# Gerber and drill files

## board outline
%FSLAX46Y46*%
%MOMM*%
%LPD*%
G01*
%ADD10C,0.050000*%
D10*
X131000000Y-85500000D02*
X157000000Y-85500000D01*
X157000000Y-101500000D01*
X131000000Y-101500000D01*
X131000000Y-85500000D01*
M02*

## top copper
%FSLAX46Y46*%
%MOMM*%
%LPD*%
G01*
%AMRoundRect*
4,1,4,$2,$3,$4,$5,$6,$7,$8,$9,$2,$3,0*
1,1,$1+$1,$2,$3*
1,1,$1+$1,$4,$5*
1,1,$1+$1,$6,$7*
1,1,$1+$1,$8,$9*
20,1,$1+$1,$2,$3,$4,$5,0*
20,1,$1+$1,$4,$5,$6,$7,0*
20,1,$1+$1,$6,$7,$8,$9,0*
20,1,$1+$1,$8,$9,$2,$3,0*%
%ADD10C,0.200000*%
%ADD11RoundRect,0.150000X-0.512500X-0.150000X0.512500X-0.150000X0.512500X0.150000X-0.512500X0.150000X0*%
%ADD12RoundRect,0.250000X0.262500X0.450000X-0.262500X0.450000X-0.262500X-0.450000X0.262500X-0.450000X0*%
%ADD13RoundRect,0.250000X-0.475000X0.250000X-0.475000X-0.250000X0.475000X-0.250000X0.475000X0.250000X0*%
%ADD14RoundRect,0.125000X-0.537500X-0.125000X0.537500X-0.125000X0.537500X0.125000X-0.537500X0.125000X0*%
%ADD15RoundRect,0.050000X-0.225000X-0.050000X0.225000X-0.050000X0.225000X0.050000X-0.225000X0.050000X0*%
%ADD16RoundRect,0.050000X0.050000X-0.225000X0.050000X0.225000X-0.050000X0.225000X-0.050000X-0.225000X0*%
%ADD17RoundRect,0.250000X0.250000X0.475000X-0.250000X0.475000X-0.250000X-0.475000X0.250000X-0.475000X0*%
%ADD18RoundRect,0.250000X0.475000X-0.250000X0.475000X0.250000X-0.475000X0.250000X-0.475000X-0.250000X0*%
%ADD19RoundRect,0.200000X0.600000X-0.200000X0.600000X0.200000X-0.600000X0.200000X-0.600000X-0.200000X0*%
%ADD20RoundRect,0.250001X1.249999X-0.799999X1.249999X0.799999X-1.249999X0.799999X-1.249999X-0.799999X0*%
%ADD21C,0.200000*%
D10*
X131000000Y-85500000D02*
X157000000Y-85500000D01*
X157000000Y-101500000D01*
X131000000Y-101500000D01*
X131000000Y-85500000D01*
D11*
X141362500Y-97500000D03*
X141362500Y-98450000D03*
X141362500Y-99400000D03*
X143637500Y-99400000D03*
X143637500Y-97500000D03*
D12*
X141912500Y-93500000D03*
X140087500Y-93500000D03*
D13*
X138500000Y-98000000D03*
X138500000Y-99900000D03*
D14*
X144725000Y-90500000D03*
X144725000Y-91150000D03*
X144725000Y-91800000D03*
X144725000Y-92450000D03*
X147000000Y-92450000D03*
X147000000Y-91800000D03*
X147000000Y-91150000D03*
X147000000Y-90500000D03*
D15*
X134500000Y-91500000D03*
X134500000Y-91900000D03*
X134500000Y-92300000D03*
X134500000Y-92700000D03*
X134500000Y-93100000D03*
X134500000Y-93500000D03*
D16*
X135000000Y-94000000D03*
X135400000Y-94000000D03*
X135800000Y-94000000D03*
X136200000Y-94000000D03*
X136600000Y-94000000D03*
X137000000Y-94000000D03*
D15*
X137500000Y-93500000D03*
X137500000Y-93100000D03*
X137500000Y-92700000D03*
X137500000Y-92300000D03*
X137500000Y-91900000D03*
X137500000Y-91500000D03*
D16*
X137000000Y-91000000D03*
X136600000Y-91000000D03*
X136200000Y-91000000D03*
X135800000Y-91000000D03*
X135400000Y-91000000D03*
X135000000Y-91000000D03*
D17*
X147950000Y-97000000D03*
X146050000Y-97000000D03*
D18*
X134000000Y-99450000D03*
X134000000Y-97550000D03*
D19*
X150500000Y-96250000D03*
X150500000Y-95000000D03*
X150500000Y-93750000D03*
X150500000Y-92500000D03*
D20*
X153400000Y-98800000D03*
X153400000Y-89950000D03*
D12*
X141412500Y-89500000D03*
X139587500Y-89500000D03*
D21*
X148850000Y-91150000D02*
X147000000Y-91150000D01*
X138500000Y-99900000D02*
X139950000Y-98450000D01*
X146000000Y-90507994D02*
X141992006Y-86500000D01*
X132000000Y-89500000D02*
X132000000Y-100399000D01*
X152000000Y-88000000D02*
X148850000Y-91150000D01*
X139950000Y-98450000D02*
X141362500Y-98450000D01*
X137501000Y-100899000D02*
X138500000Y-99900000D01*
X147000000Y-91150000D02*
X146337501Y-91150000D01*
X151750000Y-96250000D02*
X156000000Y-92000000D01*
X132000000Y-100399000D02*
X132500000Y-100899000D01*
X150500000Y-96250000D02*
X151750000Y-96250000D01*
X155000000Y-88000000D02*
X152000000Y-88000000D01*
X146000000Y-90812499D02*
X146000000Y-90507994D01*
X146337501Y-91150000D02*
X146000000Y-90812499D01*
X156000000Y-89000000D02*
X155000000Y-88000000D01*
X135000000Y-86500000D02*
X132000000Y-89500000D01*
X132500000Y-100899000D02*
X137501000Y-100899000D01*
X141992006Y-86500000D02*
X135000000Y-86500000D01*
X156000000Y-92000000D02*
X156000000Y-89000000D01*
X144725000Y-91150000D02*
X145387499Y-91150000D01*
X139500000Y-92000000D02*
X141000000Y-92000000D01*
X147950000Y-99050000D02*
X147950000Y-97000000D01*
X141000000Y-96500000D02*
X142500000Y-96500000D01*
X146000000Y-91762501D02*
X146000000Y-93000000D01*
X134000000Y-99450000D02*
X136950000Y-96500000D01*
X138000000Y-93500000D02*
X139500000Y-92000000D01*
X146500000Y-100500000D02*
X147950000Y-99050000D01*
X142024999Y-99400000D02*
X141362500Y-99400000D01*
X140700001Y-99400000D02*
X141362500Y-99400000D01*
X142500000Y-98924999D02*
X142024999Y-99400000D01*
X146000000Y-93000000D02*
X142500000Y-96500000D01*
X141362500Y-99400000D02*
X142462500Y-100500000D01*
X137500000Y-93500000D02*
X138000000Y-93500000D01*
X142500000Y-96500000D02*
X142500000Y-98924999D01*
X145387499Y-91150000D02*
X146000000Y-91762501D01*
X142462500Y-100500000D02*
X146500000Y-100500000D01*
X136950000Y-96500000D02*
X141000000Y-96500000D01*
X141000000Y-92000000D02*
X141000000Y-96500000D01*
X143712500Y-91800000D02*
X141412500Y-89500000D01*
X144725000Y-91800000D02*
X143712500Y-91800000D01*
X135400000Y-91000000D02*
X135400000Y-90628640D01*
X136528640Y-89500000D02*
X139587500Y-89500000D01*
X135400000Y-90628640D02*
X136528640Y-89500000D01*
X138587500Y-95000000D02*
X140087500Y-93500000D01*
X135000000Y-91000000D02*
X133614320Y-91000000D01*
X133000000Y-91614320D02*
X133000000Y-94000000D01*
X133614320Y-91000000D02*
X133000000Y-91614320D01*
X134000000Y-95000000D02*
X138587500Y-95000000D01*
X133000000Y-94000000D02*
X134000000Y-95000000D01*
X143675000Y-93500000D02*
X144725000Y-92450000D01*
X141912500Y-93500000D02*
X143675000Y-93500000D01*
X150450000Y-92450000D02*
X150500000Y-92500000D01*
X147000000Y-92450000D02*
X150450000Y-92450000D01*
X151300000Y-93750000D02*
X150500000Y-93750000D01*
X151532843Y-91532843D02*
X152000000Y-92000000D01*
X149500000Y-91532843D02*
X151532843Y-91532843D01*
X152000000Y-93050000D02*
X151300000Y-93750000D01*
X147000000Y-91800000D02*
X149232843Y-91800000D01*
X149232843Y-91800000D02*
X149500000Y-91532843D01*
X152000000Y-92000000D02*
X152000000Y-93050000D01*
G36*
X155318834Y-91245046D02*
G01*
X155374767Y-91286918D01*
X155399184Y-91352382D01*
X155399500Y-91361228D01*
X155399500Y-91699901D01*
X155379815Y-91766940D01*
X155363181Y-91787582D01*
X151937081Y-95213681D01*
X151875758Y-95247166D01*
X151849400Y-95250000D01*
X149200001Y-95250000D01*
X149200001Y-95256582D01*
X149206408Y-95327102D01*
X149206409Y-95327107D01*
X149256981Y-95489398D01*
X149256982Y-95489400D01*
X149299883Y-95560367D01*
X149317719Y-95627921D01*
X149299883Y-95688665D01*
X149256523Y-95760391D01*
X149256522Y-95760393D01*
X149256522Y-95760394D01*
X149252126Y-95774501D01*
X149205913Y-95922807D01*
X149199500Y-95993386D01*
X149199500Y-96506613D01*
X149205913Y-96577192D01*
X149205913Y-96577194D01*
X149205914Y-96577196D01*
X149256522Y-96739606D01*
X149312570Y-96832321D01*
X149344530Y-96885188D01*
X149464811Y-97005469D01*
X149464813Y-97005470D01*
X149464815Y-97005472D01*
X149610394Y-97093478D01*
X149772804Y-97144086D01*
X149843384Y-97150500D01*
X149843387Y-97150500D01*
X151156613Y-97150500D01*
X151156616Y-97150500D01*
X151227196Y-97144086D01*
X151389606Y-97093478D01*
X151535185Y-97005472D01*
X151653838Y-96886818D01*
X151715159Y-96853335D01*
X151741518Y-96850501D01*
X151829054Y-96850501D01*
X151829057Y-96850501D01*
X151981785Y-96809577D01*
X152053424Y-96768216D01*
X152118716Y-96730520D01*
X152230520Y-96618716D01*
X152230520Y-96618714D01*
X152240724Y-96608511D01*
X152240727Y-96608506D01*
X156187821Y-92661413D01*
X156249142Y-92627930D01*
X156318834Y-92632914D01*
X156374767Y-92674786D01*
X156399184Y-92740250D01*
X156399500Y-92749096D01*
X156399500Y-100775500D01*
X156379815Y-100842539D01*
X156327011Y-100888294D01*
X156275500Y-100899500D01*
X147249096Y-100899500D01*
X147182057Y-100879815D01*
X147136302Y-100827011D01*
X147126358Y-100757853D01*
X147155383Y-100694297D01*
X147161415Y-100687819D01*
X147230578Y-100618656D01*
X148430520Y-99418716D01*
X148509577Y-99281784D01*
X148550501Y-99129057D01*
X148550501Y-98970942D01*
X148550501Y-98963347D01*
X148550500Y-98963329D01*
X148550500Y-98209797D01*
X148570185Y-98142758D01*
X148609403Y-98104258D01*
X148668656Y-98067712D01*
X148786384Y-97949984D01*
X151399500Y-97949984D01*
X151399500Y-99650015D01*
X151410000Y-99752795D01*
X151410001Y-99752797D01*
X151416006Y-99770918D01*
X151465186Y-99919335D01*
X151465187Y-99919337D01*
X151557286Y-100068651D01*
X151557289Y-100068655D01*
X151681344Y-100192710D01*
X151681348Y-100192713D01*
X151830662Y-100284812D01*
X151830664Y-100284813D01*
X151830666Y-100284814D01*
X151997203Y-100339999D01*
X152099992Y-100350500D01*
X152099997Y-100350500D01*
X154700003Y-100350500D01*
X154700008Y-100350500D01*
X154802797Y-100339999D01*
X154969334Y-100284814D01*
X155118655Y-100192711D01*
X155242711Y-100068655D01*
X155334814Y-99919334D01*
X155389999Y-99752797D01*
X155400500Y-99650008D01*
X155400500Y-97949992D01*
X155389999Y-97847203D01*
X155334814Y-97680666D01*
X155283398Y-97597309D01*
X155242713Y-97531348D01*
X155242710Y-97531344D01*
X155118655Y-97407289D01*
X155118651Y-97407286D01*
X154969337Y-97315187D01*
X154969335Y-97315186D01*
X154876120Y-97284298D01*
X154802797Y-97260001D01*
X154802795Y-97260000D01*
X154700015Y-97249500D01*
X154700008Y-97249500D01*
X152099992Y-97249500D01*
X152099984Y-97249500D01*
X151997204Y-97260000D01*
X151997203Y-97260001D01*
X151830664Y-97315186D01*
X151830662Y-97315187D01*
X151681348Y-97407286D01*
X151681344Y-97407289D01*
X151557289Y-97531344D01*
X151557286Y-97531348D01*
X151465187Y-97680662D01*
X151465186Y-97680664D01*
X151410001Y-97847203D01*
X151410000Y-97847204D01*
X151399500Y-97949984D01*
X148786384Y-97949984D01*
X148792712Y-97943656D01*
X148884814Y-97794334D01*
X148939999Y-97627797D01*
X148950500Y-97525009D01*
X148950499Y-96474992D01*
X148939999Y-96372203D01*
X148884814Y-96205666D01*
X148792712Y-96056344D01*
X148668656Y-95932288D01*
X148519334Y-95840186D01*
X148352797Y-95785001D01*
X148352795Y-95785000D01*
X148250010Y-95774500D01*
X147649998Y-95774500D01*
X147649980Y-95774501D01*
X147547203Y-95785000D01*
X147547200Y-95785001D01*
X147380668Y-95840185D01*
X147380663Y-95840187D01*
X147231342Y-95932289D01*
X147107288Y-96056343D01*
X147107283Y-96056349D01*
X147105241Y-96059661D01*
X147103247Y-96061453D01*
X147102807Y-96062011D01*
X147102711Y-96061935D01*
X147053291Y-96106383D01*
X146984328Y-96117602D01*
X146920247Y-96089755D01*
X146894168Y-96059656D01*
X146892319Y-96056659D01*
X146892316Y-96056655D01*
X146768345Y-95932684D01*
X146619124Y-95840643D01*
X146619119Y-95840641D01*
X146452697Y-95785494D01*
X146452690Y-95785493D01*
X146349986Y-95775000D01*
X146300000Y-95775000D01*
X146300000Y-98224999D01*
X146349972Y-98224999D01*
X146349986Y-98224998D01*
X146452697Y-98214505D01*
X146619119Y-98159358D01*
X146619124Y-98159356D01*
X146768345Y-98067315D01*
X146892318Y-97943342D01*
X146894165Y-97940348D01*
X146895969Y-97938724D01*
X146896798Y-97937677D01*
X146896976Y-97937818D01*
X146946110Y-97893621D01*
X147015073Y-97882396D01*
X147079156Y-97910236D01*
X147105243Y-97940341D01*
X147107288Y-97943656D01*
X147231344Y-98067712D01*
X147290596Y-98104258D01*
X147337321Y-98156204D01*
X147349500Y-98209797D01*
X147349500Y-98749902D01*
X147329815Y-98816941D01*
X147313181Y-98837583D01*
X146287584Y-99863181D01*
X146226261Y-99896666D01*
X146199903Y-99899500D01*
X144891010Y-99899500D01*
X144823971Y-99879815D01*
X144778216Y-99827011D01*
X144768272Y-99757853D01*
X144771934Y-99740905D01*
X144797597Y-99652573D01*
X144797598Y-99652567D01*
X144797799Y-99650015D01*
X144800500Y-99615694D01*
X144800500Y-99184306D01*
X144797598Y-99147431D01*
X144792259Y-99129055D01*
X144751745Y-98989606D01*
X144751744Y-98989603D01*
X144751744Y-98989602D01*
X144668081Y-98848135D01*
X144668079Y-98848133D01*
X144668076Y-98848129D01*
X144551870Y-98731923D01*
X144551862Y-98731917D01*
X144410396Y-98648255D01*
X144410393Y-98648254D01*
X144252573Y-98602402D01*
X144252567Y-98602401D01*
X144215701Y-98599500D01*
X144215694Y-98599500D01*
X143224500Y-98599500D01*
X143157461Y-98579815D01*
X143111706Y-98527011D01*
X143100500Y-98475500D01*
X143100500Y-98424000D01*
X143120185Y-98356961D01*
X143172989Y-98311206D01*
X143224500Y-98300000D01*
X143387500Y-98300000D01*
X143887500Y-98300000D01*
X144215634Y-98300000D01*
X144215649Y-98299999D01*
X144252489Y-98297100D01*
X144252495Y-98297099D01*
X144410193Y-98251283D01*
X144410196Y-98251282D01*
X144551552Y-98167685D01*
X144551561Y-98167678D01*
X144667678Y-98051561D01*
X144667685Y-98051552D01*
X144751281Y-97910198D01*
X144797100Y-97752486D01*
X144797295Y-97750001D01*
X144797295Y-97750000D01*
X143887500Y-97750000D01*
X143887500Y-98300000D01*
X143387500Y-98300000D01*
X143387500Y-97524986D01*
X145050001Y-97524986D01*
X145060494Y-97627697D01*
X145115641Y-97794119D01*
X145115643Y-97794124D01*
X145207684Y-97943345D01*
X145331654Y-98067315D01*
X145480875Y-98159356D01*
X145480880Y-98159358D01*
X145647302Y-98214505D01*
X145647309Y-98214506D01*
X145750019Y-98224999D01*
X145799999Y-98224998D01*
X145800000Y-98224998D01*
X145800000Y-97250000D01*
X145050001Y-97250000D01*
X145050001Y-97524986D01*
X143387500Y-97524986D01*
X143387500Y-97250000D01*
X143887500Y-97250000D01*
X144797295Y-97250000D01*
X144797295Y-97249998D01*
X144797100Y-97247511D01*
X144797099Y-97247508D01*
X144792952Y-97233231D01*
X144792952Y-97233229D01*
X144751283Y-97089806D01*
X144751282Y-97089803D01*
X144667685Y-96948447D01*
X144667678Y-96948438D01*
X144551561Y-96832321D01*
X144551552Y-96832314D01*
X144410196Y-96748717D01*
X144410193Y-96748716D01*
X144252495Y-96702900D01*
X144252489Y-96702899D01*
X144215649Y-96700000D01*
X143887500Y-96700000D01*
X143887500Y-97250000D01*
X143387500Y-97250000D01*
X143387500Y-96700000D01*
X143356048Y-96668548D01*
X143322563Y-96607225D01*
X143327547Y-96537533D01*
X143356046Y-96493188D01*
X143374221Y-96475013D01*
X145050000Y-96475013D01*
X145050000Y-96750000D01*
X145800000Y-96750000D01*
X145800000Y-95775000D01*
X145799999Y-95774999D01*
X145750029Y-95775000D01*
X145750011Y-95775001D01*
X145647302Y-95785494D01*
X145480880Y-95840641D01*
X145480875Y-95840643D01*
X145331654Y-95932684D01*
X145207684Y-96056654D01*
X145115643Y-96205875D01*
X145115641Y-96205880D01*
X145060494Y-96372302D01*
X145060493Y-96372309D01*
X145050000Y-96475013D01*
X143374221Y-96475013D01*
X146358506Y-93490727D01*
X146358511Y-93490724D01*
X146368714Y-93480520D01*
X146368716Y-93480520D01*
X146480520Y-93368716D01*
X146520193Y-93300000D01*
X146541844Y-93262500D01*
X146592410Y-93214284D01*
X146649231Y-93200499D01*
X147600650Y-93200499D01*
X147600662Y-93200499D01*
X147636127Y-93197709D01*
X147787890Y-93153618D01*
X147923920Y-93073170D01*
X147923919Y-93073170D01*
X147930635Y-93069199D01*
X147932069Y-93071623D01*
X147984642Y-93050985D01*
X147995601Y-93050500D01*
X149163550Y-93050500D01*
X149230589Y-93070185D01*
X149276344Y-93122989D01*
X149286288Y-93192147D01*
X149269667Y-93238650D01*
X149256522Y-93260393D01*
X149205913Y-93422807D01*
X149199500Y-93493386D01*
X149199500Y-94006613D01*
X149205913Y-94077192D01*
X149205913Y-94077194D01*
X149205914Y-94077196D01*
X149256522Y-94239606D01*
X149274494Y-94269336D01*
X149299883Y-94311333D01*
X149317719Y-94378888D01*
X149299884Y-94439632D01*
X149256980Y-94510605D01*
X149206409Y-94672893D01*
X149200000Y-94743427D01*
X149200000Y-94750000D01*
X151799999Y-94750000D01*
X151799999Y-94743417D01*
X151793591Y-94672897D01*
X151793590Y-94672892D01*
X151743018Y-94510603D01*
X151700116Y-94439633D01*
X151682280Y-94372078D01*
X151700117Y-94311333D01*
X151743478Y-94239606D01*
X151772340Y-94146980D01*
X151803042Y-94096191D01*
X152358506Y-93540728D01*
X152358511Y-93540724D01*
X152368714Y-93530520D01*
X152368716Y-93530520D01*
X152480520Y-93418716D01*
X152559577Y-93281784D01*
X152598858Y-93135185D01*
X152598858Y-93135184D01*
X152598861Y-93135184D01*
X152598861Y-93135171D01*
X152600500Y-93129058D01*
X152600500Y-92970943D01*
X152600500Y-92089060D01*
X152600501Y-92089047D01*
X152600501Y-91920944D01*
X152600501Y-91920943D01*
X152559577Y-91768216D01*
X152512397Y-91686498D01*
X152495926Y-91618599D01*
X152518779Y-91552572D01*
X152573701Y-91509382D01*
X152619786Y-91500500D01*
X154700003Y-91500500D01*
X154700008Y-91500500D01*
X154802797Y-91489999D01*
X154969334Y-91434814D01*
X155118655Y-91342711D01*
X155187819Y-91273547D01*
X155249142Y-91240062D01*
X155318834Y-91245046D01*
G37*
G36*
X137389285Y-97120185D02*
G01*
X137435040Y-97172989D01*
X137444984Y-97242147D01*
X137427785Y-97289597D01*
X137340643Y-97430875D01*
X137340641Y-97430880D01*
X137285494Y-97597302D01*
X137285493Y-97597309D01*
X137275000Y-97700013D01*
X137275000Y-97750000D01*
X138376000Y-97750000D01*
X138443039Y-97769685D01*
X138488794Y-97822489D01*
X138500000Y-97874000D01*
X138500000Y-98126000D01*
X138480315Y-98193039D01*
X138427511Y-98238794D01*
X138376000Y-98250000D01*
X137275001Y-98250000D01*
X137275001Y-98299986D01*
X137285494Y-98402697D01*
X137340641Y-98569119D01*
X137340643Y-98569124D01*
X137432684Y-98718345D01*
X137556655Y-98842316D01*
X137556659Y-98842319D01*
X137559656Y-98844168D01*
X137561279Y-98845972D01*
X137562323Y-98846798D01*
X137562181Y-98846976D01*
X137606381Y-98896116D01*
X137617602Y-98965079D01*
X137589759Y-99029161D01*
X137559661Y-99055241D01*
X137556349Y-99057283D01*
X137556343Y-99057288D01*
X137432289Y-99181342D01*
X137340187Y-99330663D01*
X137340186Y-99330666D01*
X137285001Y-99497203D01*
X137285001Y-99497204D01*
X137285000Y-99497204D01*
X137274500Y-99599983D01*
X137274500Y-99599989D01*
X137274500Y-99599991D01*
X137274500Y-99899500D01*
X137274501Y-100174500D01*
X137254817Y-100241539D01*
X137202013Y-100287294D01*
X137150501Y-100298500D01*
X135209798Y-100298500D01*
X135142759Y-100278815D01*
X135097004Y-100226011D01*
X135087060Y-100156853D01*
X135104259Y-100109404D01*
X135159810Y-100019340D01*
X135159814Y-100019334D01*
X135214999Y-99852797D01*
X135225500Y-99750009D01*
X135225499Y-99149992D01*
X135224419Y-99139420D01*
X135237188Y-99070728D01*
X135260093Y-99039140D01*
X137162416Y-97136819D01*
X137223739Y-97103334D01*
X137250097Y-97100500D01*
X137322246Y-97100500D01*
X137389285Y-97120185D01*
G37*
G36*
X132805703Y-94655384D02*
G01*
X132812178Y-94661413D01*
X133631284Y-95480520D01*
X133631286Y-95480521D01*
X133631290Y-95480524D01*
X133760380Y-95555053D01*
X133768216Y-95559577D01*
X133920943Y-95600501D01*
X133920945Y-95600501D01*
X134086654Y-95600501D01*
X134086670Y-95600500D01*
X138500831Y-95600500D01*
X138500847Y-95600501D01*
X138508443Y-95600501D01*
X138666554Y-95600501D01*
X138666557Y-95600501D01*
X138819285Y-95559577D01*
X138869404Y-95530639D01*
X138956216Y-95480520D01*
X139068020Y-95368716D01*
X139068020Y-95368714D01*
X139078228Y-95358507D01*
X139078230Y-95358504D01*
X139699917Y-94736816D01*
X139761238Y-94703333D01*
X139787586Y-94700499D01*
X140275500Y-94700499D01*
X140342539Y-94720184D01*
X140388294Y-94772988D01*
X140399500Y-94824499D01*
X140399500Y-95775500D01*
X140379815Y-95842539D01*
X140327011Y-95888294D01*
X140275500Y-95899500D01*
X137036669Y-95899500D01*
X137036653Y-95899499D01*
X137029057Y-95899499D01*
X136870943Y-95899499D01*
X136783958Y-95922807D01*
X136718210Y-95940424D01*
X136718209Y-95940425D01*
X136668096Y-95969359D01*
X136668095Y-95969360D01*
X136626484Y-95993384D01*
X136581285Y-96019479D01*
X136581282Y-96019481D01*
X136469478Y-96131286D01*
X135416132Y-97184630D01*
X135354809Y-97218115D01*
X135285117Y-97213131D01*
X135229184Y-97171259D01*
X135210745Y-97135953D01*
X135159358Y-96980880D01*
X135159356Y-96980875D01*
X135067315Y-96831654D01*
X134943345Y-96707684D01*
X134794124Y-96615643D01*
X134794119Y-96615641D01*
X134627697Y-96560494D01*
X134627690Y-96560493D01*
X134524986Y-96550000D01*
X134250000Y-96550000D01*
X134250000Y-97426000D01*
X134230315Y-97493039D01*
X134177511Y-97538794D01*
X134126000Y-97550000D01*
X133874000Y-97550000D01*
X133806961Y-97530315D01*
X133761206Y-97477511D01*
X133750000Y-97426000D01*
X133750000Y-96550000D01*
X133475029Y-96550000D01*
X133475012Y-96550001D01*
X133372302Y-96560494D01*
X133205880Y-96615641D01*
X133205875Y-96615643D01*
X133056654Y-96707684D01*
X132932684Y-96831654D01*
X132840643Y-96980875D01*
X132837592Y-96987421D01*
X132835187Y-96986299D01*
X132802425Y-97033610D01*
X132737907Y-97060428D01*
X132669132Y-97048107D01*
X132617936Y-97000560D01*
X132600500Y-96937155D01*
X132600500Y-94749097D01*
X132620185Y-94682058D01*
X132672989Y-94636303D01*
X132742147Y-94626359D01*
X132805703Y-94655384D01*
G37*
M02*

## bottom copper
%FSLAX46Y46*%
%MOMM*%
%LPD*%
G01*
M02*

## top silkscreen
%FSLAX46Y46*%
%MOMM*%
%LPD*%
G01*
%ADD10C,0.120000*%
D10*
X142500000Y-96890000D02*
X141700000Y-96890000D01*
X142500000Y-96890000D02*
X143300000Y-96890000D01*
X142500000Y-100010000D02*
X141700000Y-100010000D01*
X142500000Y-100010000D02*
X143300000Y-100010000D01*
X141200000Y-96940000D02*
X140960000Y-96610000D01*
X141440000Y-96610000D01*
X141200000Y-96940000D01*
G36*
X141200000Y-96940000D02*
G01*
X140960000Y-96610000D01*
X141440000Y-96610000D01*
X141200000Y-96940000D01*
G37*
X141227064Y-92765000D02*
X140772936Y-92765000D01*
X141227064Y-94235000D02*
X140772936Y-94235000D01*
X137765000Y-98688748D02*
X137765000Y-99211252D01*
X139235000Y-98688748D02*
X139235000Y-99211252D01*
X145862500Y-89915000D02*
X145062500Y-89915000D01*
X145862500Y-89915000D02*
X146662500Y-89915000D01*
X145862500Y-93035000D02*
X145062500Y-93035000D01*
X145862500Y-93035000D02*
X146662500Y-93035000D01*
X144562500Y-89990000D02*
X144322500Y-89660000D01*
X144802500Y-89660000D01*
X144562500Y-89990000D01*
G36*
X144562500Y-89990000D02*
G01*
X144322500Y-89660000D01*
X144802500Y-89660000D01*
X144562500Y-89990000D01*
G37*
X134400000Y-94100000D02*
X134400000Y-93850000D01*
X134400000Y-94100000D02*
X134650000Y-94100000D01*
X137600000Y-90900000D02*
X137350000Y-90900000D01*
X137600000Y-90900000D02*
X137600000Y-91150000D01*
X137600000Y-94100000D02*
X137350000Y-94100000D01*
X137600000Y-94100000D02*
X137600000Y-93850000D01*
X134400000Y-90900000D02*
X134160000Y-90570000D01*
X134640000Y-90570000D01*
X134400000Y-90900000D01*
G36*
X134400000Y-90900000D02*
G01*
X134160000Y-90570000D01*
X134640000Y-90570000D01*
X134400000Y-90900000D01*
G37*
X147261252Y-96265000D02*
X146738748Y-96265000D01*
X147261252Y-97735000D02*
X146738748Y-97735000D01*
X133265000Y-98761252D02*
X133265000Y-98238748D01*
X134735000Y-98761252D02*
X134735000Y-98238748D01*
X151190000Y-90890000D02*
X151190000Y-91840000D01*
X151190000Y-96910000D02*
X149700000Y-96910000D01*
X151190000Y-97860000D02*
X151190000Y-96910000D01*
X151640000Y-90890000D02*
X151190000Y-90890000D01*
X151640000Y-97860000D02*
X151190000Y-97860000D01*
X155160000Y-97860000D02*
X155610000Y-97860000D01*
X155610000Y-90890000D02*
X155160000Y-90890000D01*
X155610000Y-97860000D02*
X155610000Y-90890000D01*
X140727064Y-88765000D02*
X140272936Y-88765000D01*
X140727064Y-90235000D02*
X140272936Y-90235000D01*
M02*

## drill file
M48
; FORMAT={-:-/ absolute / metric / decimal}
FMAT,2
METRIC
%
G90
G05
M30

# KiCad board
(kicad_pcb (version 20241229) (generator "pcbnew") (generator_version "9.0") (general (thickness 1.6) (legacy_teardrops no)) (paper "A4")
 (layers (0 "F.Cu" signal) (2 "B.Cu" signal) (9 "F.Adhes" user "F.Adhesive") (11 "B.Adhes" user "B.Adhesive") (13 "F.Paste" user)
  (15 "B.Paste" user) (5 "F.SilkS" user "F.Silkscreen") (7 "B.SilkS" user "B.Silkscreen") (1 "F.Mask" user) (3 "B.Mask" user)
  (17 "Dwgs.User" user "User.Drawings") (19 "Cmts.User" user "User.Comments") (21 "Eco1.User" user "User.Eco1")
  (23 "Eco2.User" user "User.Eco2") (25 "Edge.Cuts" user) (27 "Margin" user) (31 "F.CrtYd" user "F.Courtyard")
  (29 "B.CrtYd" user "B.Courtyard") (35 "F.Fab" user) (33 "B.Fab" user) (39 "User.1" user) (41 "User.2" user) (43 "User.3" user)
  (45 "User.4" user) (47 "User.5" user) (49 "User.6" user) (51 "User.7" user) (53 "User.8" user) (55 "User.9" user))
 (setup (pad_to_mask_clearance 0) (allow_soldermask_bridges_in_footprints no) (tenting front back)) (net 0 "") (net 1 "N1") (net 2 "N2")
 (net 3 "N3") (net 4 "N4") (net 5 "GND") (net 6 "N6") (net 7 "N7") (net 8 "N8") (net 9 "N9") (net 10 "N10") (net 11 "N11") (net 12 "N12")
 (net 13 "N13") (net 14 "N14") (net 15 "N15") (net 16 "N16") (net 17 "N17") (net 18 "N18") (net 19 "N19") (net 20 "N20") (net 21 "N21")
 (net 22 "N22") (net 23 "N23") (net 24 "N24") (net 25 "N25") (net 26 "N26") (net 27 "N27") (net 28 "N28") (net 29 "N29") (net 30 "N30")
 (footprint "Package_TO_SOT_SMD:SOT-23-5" (layer "F.Cu") (at 142.5 98.45)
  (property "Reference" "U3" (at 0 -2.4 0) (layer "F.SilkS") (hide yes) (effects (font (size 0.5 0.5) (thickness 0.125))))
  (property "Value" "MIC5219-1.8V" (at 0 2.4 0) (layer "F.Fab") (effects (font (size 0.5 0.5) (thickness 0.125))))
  (fp_line (start 0 -1.56) (end -0.8 -1.56) (stroke (width 0.12) (type solid)) (layer "F.SilkS"))
  (fp_line (start 0 -1.56) (end 0.8 -1.56) (stroke (width 0.12) (type solid)) (layer "F.SilkS"))
  (fp_line (start 0 1.56) (end -0.8 1.56) (stroke (width 0.12) (type solid)) (layer "F.SilkS"))
  (fp_line (start 0 1.56) (end 0.8 1.56) (stroke (width 0.12) (type solid)) (layer "F.SilkS"))
  (fp_poly
   (pts (xy -1.3 -1.51) (xy -1.54 -1.84) (xy -1.06 -1.84) (xy -1.3 -1.51)) (stroke (width 0.12) (type solid)) (fill yes) (layer "F.SilkS"))
  (pad "1" smd roundrect (at -1.1375 -0.95) (size 1.325 0.6) (layers "F.Cu" "F.Mask" "F.Paste") (roundrect_rratio 0.25) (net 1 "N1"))
  (pad "2" smd roundrect (at -1.1375 0) (size 1.325 0.6) (layers "F.Cu" "F.Mask" "F.Paste") (roundrect_rratio 0.25) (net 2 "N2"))
  (pad "3" smd roundrect (at -1.1375 0.95) (size 1.325 0.6) (layers "F.Cu" "F.Mask" "F.Paste") (roundrect_rratio 0.25) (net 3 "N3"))
  (pad "4" smd roundrect (at 1.1375 0.95) (size 1.325 0.6) (layers "F.Cu" "F.Mask" "F.Paste") (roundrect_rratio 0.25) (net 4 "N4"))
  (pad "5" smd roundrect (at 1.1375 -0.95) (size 1.325 0.6) (layers "F.Cu" "F.Mask" "F.Paste") (roundrect_rratio 0.25) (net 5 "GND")))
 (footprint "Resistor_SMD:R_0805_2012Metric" (layer "F.Cu") (at 141 93.5 180)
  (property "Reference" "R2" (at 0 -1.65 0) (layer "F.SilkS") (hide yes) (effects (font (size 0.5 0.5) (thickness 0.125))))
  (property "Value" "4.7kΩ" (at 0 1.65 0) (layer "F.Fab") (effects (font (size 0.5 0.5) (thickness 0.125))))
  (fp_line (start -0.227064 0.735) (end 0.227064 0.735) (stroke (width 0.12) (type solid)) (layer "F.SilkS"))
  (fp_line (start -0.227064 -0.735) (end 0.227064 -0.735) (stroke (width 0.12) (type solid)) (layer "F.SilkS"))
  (pad "1" smd roundrect (at -0.9125 0 180) (size 1.025 1.4) (layers "F.Cu" "F.Mask" "F.Paste") (roundrect_rratio 0.243902) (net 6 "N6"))
  (pad "2" smd roundrect (at 0.9125 0 180) (size 1.025 1.4) (layers "F.Cu" "F.Mask" "F.Paste") (roundrect_rratio 0.243902) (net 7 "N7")))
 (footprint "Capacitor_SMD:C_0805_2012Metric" (layer "F.Cu") (at 138.5 98.95 -90)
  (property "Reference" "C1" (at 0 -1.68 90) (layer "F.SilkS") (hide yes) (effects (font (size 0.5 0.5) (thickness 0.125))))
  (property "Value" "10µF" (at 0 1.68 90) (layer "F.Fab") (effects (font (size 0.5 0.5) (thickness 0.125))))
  (fp_line (start -0.261252 0.735) (end 0.261252 0.735) (stroke (width 0.12) (type solid)) (layer "F.SilkS"))
  (fp_line (start -0.261252 -0.735) (end 0.261252 -0.735) (stroke (width 0.12) (type solid)) (layer "F.SilkS"))
  (pad "1" smd roundrect (at -0.95 0 270) (size 1 1.45) (layers "F.Cu" "F.Mask" "F.Paste") (roundrect_rratio 0.25) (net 5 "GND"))
  (pad "2" smd roundrect (at 0.95 0 270) (size 1 1.45) (layers "F.Cu" "F.Mask" "F.Paste") (roundrect_rratio 0.25) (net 2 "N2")))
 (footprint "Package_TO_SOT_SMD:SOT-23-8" (layer "F.Cu") (at 145.8625 91.475)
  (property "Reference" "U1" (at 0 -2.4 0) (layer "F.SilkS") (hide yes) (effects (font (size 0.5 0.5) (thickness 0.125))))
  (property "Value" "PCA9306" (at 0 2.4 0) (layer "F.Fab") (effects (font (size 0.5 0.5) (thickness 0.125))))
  (fp_line (start 0 -1.56) (end -0.8 -1.56) (stroke (width 0.12) (type solid)) (layer "F.SilkS"))
  (fp_line (start 0 -1.56) (end 0.8 -1.56) (stroke (width 0.12) (type solid)) (layer "F.SilkS"))
  (fp_line (start 0 1.56) (end -0.8 1.56) (stroke (width 0.12) (type solid)) (layer "F.SilkS"))
  (fp_line (start 0 1.56) (end 0.8 1.56) (stroke (width 0.12) (type solid)) (layer "F.SilkS"))
  (fp_poly
   (pts (xy -1.3 -1.485) (xy -1.54 -1.815) (xy -1.06 -1.815) (xy -1.3 -1.485)) (stroke (width 0.12) (type solid)) (fill yes)
   (layer "F.SilkS"))
  (pad "1" smd roundrect (at -1.1375 -0.975) (size 1.325 0.5) (layers "F.Cu" "F.Mask" "F.Paste") (roundrect_rratio 0.25) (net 5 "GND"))
  (pad "2" smd roundrect (at -1.1375 -0.325) (size 1.325 0.5) (layers "F.Cu" "F.Mask" "F.Paste") (roundrect_rratio 0.25) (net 3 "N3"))
  (pad "3" smd roundrect (at -1.1375 0.325) (size 1.325 0.5) (layers "F.Cu" "F.Mask" "F.Paste") (roundrect_rratio 0.25) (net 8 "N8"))
  (pad "4" smd roundrect (at -1.1375 0.975) (size 1.325 0.5) (layers "F.Cu" "F.Mask" "F.Paste") (roundrect_rratio 0.25) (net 6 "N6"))
  (pad "5" smd roundrect (at 1.1375 0.975) (size 1.325 0.5) (layers "F.Cu" "F.Mask" "F.Paste") (roundrect_rratio 0.25) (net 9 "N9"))
  (pad "6" smd roundrect (at 1.1375 0.325) (size 1.325 0.5) (layers "F.Cu" "F.Mask" "F.Paste") (roundrect_rratio 0.25) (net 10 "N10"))
  (pad "7" smd roundrect (at 1.1375 -0.325) (size 1.325 0.5) (layers "F.Cu" "F.Mask" "F.Paste") (roundrect_rratio 0.25) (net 2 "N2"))
  (pad "8" smd roundrect (at 1.1375 -0.975) (size 1.325 0.5) (layers "F.Cu" "F.Mask" "F.Paste") (roundrect_rratio 0.25) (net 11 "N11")))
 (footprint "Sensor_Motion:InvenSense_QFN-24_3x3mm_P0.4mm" (layer "F.Cu") (at 136 92.5)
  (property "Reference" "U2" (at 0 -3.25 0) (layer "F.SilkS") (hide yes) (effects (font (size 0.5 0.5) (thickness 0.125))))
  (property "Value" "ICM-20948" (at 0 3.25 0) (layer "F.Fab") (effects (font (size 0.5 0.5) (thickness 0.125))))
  (fp_line (start -1.6 1.6) (end -1.6 1.35) (stroke (width 0.12) (type solid)) (layer "F.SilkS"))
  (fp_line (start -1.6 1.6) (end -1.35 1.6) (stroke (width 0.12) (type solid)) (layer "F.SilkS"))
  (fp_line (start 1.6 -1.6) (end 1.35 -1.6) (stroke (width 0.12) (type solid)) (layer "F.SilkS"))
  (fp_line (start 1.6 -1.6) (end 1.6 -1.35) (stroke (width 0.12) (type solid)) (layer "F.SilkS"))
  (fp_line (start 1.6 1.6) (end 1.35 1.6) (stroke (width 0.12) (type solid)) (layer "F.SilkS"))
  (fp_line (start 1.6 1.6) (end 1.6 1.35) (stroke (width 0.12) (type solid)) (layer "F.SilkS"))
  (fp_poly
   (pts (xy -1.6 -1.6) (xy -1.84 -1.93) (xy -1.36 -1.93) (xy -1.6 -1.6)) (stroke (width 0.12) (type solid)) (fill yes) (layer "F.SilkS"))
  (pad "1" smd roundrect (at -1.5 -1) (size 0.55 0.2) (layers "F.Cu" "F.Mask" "F.Paste") (roundrect_rratio 0.25) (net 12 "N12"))
  (pad "2" smd roundrect (at -1.5 -0.6) (size 0.55 0.2) (layers "F.Cu" "F.Mask" "F.Paste") (roundrect_rratio 0.25) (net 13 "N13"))
  (pad "3" smd roundrect (at -1.5 -0.2) (size 0.55 0.2) (layers "F.Cu" "F.Mask" "F.Paste") (roundrect_rratio 0.25) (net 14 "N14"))
  (pad "4" smd roundrect (at -1.5 0.2) (size 0.55 0.2) (layers "F.Cu" "F.Mask" "F.Paste") (roundrect_rratio 0.25) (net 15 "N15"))
  (pad "5" smd roundrect (at -1.5 0.6) (size 0.55 0.2) (layers "F.Cu" "F.Mask" "F.Paste") (roundrect_rratio 0.25) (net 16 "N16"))
  (pad "6" smd roundrect (at -1.5 1) (size 0.55 0.2) (layers "F.Cu" "F.Mask" "F.Paste") (roundrect_rratio 0.25) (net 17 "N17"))
  (pad "7" smd roundrect (at -1 1.5 90) (size 0.55 0.2) (layers "F.Cu" "F.Mask" "F.Paste") (roundrect_rratio 0.25) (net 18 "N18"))
  (pad "8" smd roundrect (at -0.6 1.5 90) (size 0.55 0.2) (layers "F.Cu" "F.Mask" "F.Paste") (roundrect_rratio 0.25) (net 3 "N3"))
  (pad "9" smd roundrect (at -0.2 1.5 90) (size 0.55 0.2) (layers "F.Cu" "F.Mask" "F.Paste") (roundrect_rratio 0.25) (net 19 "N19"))
  (pad "10" smd roundrect (at 0.2 1.5 90) (size 0.55 0.2) (layers "F.Cu" "F.Mask" "F.Paste") (roundrect_rratio 0.25) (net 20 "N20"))
  (pad "11" smd roundrect (at 0.6 1.5 90) (size 0.55 0.2) (layers "F.Cu" "F.Mask" "F.Paste") (roundrect_rratio 0.25) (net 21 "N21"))
  (pad "12" smd roundrect (at 1 1.5 90) (size 0.55 0.2) (layers "F.Cu" "F.Mask" "F.Paste") (roundrect_rratio 0.25) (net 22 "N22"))
  (pad "13" smd roundrect (at 1.5 1) (size 0.55 0.2) (layers "F.Cu" "F.Mask" "F.Paste") (roundrect_rratio 0.25) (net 3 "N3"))
  (pad "14" smd roundrect (at 1.5 0.6) (size 0.55 0.2) (layers "F.Cu" "F.Mask" "F.Paste") (roundrect_rratio 0.25) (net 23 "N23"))
  (pad "15" smd roundrect (at 1.5 0.2) (size 0.55 0.2) (layers "F.Cu" "F.Mask" "F.Paste") (roundrect_rratio 0.25) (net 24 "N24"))
  (pad "16" smd roundrect (at 1.5 -0.2) (size 0.55 0.2) (layers "F.Cu" "F.Mask" "F.Paste") (roundrect_rratio 0.25) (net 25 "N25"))
  (pad "17" smd roundrect (at 1.5 -0.6) (size 0.55 0.2) (layers "F.Cu" "F.Mask" "F.Paste") (roundrect_rratio 0.25) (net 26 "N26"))
  (pad "18" smd roundrect (at 1.5 -1) (size 0.55 0.2) (layers "F.Cu" "F.Mask" "F.Paste") (roundrect_rratio 0.25) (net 5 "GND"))
  (pad "19" smd roundrect (at 1 -1.5 90) (size 0.55 0.2) (layers "F.Cu" "F.Mask" "F.Paste") (roundrect_rratio 0.25) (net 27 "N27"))
  (pad "20" smd roundrect (at 0.6 -1.5 90) (size 0.55 0.2) (layers "F.Cu" "F.Mask" "F.Paste") (roundrect_rratio 0.25) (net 5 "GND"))
  (pad "21" smd roundrect (at 0.2 -1.5 90) (size 0.55 0.2) (layers "F.Cu" "F.Mask" "F.Paste") (roundrect_rratio 0.25) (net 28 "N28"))
  (pad "22" smd roundrect (at -0.2 -1.5 90) (size 0.55 0.2) (layers "F.Cu" "F.Mask" "F.Paste") (roundrect_rratio 0.25) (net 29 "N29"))
  (pad "23" smd roundrect (at -0.6 -1.5 90) (size 0.55 0.2) (layers "F.Cu" "F.Mask" "F.Paste") (roundrect_rratio 0.25) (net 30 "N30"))
  (pad "24" smd roundrect (at -1 -1.5 90) (size 0.55 0.2) (layers "F.Cu" "F.Mask" "F.Paste") (roundrect_rratio 0.25) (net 7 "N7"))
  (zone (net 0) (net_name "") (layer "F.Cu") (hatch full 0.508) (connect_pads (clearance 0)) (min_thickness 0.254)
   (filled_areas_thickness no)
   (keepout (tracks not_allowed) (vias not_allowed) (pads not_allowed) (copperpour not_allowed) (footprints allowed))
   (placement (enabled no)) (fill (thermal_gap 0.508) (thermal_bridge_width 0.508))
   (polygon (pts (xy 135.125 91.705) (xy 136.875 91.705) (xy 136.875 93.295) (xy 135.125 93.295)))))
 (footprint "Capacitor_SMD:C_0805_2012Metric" (layer "F.Cu") (at 147 97 180)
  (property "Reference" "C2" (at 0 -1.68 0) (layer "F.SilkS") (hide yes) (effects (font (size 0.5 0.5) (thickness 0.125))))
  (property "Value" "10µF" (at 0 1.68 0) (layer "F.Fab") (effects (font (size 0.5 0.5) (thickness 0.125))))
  (fp_line (start -0.261252 0.735) (end 0.261252 0.735) (stroke (width 0.12) (type solid)) (layer "F.SilkS"))
  (fp_line (start -0.261252 -0.735) (end 0.261252 -0.735) (stroke (width 0.12) (type solid)) (layer "F.SilkS"))
  (pad "1" smd roundrect (at -0.95 0 180) (size 1 1.45) (layers "F.Cu" "F.Mask" "F.Paste") (roundrect_rratio 0.25) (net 3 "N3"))
  (pad "2" smd roundrect (at 0.95 0 180) (size 1 1.45) (layers "F.Cu" "F.Mask" "F.Paste") (roundrect_rratio 0.25) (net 5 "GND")))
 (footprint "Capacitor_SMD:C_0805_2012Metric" (layer "F.Cu") (at 134 98.5 90)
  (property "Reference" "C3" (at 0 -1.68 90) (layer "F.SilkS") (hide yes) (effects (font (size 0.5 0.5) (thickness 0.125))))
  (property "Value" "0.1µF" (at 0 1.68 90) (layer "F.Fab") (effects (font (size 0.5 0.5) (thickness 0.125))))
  (fp_line (start -0.261252 -0.735) (end 0.261252 -0.735) (stroke (width 0.12) (type solid)) (layer "F.SilkS"))
  (fp_line (start -0.261252 0.735) (end 0.261252 0.735) (stroke (width 0.12) (type solid)) (layer "F.SilkS"))
  (pad "1" smd roundrect (at -0.95 0 90) (size 1 1.45) (layers "F.Cu" "F.Mask" "F.Paste") (roundrect_rratio 0.25) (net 3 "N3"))
  (pad "2" smd roundrect (at 0.95 0 90) (size 1 1.45) (layers "F.Cu" "F.Mask" "F.Paste") (roundrect_rratio 0.25) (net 5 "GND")))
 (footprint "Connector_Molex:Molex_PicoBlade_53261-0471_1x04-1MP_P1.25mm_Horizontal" (layer "F.Cu") (at 152.9 94.375 90)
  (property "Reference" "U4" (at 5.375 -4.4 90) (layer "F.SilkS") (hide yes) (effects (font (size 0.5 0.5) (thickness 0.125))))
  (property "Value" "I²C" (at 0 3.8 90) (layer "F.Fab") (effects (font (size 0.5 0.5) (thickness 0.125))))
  (fp_line (start 3.485 -1.71) (end 2.535 -1.71) (stroke (width 0.12) (type solid)) (layer "F.SilkS"))
  (fp_line (start -2.535 -1.71) (end -2.535 -3.2) (stroke (width 0.12) (type solid)) (layer "F.SilkS"))
  (fp_line (start -3.485 -1.71) (end -2.535 -1.71) (stroke (width 0.12) (type solid)) (layer "F.SilkS"))
  (fp_line (start 3.485 -1.26) (end 3.485 -1.71) (stroke (width 0.12) (type solid)) (layer "F.SilkS"))
  (fp_line (start -3.485 -1.26) (end -3.485 -1.71) (stroke (width 0.12) (type solid)) (layer "F.SilkS"))
  (fp_line (start -3.485 2.26) (end -3.485 2.71) (stroke (width 0.12) (type solid)) (layer "F.SilkS"))
  (fp_line (start 3.485 2.71) (end 3.485 2.26) (stroke (width 0.12) (type solid)) (layer "F.SilkS"))
  (fp_line (start -3.485 2.71) (end 3.485 2.71) (stroke (width 0.12) (type solid)) (layer "F.SilkS"))
  (pad "1" smd roundrect (at -1.875 -2.4 90) (size 0.8 1.6) (layers "F.Cu" "F.Mask" "F.Paste") (roundrect_rratio 0.25) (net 2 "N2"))
  (pad "2" smd roundrect (at -0.625 -2.4 90) (size 0.8 1.6) (layers "F.Cu" "F.Mask" "F.Paste") (roundrect_rratio 0.25) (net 5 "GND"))
  (pad "3" smd roundrect (at 0.625 -2.4 90) (size 0.8 1.6) (layers "F.Cu" "F.Mask" "F.Paste") (roundrect_rratio 0.25) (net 10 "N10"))
  (pad "4" smd roundrect (at 1.875 -2.4 90) (size 0.8 1.6) (layers "F.Cu" "F.Mask" "F.Paste") (roundrect_rratio 0.25) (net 9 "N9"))
  (pad "MP" smd roundrect (at -4.425 0.5 90) (size 2.1 3) (layers "F.Cu" "F.Mask" "F.Paste") (roundrect_rratio 0.119048))
  (pad "MP" smd roundrect (at 4.425 0.5 90) (size 2.1 3) (layers "F.Cu" "F.Mask" "F.Paste") (roundrect_rratio 0.119048)))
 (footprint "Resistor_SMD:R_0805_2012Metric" (layer "F.Cu") (at 140.5 89.5 180)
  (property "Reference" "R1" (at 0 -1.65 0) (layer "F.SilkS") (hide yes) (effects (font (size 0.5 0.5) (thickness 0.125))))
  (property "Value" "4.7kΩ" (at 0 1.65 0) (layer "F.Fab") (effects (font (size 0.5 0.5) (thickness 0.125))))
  (fp_line (start -0.227064 0.735) (end 0.227064 0.735) (stroke (width 0.12) (type solid)) (layer "F.SilkS"))
  (fp_line (start -0.227064 -0.735) (end 0.227064 -0.735) (stroke (width 0.12) (type solid)) (layer "F.SilkS"))
  (pad "1" smd roundrect (at -0.9125 0 180) (size 1.025 1.4) (layers "F.Cu" "F.Mask" "F.Paste") (roundrect_rratio 0.243902) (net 8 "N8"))
  (pad "2" smd roundrect (at 0.9125 0 180) (size 1.025 1.4) (layers "F.Cu" "F.Mask" "F.Paste") (roundrect_rratio 0.243902) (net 30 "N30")))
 (gr_rect (start 131 85.5) (end 157 101.5) (stroke (width 0.2) (type default)) (fill no) (layer "F.Cu"))
 (gr_rect (start 131 85.5) (end 157 101.5) (stroke (width 0.05) (type default)) (fill no) (layer "Edge.Cuts"))
 (segment (start 148.85 91.15) (end 147 91.15) (width 0.2) (layer "F.Cu") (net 2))
 (segment (start 138.5 99.9) (end 139.95 98.45) (width 0.2) (layer "F.Cu") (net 2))
 (segment (start 146 90.507994) (end 141.992006 86.5) (width 0.2) (layer "F.Cu") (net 2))
 (segment (start 132 89.5) (end 132 100.399) (width 0.2) (layer "F.Cu") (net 2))
 (segment (start 152 88) (end 148.85 91.15) (width 0.2) (layer "F.Cu") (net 2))
 (segment (start 139.95 98.45) (end 141.3625 98.45) (width 0.2) (layer "F.Cu") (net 2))
 (segment (start 137.501 100.899) (end 138.5 99.9) (width 0.2) (layer "F.Cu") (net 2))
 (segment (start 147 91.15) (end 146.337501 91.15) (width 0.2) (layer "F.Cu") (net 2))
 (segment (start 151.75 96.25) (end 156 92) (width 0.2) (layer "F.Cu") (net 2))
 (segment (start 132 100.399) (end 132.5 100.899) (width 0.2) (layer "F.Cu") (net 2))
 (segment (start 150.5 96.25) (end 151.75 96.25) (width 0.2) (layer "F.Cu") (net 2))
 (segment (start 155 88) (end 152 88) (width 0.2) (layer "F.Cu") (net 2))
 (segment (start 146 90.812499) (end 146 90.507994) (width 0.2) (layer "F.Cu") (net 2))
 (segment (start 146.337501 91.15) (end 146 90.812499) (width 0.2) (layer "F.Cu") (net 2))
 (segment (start 156 89) (end 155 88) (width 0.2) (layer "F.Cu") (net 2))
 (segment (start 135 86.5) (end 132 89.5) (width 0.2) (layer "F.Cu") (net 2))
 (segment (start 132.5 100.899) (end 137.501 100.899) (width 0.2) (layer "F.Cu") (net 2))
 (segment (start 141.992006 86.5) (end 135 86.5) (width 0.2) (layer "F.Cu") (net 2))
 (segment (start 156 92) (end 156 89) (width 0.2) (layer "F.Cu") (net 2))
 (segment (start 144.725 91.15) (end 145.387499 91.15) (width 0.2) (layer "F.Cu") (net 3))
 (segment (start 139.5 92) (end 141 92) (width 0.2) (layer "F.Cu") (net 3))
 (segment (start 147.95 99.05) (end 147.95 97) (width 0.2) (layer "F.Cu") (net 3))
 (segment (start 141 96.5) (end 142.5 96.5) (width 0.2) (layer "F.Cu") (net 3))
 (segment (start 146 91.762501) (end 146 93) (width 0.2) (layer "F.Cu") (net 3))
 (segment (start 134 99.45) (end 136.95 96.5) (width 0.2) (layer "F.Cu") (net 3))
 (segment (start 138 93.5) (end 139.5 92) (width 0.2) (layer "F.Cu") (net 3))
 (segment (start 146.5 100.5) (end 147.95 99.05) (width 0.2) (layer "F.Cu") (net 3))
 (segment (start 142.024999 99.4) (end 141.3625 99.4) (width 0.2) (layer "F.Cu") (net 3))
 (segment (start 140.700001 99.4) (end 141.3625 99.4) (width 0.2) (layer "F.Cu") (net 3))
 (segment (start 142.5 98.924999) (end 142.024999 99.4) (width 0.2) (layer "F.Cu") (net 3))
 (segment (start 146 93) (end 142.5 96.5) (width 0.2) (layer "F.Cu") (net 3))
 (segment (start 141.3625 99.4) (end 142.4625 100.5) (width 0.2) (layer "F.Cu") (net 3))
 (segment (start 137.5 93.5) (end 138 93.5) (width 0.2) (layer "F.Cu") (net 3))
 (segment (start 142.5 96.5) (end 142.5 98.924999) (width 0.2) (layer "F.Cu") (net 3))
 (segment (start 145.387499 91.15) (end 146 91.762501) (width 0.2) (layer "F.Cu") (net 3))
 (segment (start 142.4625 100.5) (end 146.5 100.5) (width 0.2) (layer "F.Cu") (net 3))
 (segment (start 136.95 96.5) (end 141 96.5) (width 0.2) (layer "F.Cu") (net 3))
 (segment (start 141 92) (end 141 96.5) (width 0.2) (layer "F.Cu") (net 3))
 (segment (start 143.7125 91.8) (end 141.4125 89.5) (width 0.2) (layer "F.Cu") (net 8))
 (segment (start 144.725 91.8) (end 143.7125 91.8) (width 0.2) (layer "F.Cu") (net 8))
 (segment (start 135.4 91) (end 135.4 90.62864) (width 0.2) (layer "F.Cu") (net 30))
 (segment (start 136.52864 89.5) (end 139.5875 89.5) (width 0.2) (layer "F.Cu") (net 30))
 (segment (start 135.4 90.62864) (end 136.52864 89.5) (width 0.2) (layer "F.Cu") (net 30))
 (segment (start 138.5875 95) (end 140.0875 93.5) (width 0.2) (layer "F.Cu") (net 7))
 (segment (start 135 91) (end 133.61432 91) (width 0.2) (layer "F.Cu") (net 7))
 (segment (start 133 91.61432) (end 133 94) (width 0.2) (layer "F.Cu") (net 7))
 (segment (start 133.61432 91) (end 133 91.61432) (width 0.2) (layer "F.Cu") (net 7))
 (segment (start 134 95) (end 138.5875 95) (width 0.2) (layer "F.Cu") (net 7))
 (segment (start 133 94) (end 134 95) (width 0.2) (layer "F.Cu") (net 7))
 (segment (start 143.675 93.5) (end 144.725 92.45) (width 0.2) (layer "F.Cu") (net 6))
 (segment (start 141.9125 93.5) (end 143.675 93.5) (width 0.2) (layer "F.Cu") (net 6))
 (segment (start 150.45 92.45) (end 150.5 92.5) (width 0.2) (layer "F.Cu") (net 9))
 (segment (start 147 92.45) (end 150.45 92.45) (width 0.2) (layer "F.Cu") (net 9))
 (segment (start 151.3 93.75) (end 150.5 93.75) (width 0.2) (layer "F.Cu") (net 10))
 (segment (start 151.532843 91.532843) (end 152 92) (width 0.2) (layer "F.Cu") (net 10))
 (segment (start 149.5 91.532843) (end 151.532843 91.532843) (width 0.2) (layer "F.Cu") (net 10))
 (segment (start 152 93.05) (end 151.3 93.75) (width 0.2) (layer "F.Cu") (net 10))
 (segment (start 147 91.8) (end 149.232843 91.8) (width 0.2) (layer "F.Cu") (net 10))
 (segment (start 149.232843 91.8) (end 149.5 91.532843) (width 0.2) (layer "F.Cu") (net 10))
 (segment (start 152 92) (end 152 93.05) (width 0.2) (layer "F.Cu") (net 10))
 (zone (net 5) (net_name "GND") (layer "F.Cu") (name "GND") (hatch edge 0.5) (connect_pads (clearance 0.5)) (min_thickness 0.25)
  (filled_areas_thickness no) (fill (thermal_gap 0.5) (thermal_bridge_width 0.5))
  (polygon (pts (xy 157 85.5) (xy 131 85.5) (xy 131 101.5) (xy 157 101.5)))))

